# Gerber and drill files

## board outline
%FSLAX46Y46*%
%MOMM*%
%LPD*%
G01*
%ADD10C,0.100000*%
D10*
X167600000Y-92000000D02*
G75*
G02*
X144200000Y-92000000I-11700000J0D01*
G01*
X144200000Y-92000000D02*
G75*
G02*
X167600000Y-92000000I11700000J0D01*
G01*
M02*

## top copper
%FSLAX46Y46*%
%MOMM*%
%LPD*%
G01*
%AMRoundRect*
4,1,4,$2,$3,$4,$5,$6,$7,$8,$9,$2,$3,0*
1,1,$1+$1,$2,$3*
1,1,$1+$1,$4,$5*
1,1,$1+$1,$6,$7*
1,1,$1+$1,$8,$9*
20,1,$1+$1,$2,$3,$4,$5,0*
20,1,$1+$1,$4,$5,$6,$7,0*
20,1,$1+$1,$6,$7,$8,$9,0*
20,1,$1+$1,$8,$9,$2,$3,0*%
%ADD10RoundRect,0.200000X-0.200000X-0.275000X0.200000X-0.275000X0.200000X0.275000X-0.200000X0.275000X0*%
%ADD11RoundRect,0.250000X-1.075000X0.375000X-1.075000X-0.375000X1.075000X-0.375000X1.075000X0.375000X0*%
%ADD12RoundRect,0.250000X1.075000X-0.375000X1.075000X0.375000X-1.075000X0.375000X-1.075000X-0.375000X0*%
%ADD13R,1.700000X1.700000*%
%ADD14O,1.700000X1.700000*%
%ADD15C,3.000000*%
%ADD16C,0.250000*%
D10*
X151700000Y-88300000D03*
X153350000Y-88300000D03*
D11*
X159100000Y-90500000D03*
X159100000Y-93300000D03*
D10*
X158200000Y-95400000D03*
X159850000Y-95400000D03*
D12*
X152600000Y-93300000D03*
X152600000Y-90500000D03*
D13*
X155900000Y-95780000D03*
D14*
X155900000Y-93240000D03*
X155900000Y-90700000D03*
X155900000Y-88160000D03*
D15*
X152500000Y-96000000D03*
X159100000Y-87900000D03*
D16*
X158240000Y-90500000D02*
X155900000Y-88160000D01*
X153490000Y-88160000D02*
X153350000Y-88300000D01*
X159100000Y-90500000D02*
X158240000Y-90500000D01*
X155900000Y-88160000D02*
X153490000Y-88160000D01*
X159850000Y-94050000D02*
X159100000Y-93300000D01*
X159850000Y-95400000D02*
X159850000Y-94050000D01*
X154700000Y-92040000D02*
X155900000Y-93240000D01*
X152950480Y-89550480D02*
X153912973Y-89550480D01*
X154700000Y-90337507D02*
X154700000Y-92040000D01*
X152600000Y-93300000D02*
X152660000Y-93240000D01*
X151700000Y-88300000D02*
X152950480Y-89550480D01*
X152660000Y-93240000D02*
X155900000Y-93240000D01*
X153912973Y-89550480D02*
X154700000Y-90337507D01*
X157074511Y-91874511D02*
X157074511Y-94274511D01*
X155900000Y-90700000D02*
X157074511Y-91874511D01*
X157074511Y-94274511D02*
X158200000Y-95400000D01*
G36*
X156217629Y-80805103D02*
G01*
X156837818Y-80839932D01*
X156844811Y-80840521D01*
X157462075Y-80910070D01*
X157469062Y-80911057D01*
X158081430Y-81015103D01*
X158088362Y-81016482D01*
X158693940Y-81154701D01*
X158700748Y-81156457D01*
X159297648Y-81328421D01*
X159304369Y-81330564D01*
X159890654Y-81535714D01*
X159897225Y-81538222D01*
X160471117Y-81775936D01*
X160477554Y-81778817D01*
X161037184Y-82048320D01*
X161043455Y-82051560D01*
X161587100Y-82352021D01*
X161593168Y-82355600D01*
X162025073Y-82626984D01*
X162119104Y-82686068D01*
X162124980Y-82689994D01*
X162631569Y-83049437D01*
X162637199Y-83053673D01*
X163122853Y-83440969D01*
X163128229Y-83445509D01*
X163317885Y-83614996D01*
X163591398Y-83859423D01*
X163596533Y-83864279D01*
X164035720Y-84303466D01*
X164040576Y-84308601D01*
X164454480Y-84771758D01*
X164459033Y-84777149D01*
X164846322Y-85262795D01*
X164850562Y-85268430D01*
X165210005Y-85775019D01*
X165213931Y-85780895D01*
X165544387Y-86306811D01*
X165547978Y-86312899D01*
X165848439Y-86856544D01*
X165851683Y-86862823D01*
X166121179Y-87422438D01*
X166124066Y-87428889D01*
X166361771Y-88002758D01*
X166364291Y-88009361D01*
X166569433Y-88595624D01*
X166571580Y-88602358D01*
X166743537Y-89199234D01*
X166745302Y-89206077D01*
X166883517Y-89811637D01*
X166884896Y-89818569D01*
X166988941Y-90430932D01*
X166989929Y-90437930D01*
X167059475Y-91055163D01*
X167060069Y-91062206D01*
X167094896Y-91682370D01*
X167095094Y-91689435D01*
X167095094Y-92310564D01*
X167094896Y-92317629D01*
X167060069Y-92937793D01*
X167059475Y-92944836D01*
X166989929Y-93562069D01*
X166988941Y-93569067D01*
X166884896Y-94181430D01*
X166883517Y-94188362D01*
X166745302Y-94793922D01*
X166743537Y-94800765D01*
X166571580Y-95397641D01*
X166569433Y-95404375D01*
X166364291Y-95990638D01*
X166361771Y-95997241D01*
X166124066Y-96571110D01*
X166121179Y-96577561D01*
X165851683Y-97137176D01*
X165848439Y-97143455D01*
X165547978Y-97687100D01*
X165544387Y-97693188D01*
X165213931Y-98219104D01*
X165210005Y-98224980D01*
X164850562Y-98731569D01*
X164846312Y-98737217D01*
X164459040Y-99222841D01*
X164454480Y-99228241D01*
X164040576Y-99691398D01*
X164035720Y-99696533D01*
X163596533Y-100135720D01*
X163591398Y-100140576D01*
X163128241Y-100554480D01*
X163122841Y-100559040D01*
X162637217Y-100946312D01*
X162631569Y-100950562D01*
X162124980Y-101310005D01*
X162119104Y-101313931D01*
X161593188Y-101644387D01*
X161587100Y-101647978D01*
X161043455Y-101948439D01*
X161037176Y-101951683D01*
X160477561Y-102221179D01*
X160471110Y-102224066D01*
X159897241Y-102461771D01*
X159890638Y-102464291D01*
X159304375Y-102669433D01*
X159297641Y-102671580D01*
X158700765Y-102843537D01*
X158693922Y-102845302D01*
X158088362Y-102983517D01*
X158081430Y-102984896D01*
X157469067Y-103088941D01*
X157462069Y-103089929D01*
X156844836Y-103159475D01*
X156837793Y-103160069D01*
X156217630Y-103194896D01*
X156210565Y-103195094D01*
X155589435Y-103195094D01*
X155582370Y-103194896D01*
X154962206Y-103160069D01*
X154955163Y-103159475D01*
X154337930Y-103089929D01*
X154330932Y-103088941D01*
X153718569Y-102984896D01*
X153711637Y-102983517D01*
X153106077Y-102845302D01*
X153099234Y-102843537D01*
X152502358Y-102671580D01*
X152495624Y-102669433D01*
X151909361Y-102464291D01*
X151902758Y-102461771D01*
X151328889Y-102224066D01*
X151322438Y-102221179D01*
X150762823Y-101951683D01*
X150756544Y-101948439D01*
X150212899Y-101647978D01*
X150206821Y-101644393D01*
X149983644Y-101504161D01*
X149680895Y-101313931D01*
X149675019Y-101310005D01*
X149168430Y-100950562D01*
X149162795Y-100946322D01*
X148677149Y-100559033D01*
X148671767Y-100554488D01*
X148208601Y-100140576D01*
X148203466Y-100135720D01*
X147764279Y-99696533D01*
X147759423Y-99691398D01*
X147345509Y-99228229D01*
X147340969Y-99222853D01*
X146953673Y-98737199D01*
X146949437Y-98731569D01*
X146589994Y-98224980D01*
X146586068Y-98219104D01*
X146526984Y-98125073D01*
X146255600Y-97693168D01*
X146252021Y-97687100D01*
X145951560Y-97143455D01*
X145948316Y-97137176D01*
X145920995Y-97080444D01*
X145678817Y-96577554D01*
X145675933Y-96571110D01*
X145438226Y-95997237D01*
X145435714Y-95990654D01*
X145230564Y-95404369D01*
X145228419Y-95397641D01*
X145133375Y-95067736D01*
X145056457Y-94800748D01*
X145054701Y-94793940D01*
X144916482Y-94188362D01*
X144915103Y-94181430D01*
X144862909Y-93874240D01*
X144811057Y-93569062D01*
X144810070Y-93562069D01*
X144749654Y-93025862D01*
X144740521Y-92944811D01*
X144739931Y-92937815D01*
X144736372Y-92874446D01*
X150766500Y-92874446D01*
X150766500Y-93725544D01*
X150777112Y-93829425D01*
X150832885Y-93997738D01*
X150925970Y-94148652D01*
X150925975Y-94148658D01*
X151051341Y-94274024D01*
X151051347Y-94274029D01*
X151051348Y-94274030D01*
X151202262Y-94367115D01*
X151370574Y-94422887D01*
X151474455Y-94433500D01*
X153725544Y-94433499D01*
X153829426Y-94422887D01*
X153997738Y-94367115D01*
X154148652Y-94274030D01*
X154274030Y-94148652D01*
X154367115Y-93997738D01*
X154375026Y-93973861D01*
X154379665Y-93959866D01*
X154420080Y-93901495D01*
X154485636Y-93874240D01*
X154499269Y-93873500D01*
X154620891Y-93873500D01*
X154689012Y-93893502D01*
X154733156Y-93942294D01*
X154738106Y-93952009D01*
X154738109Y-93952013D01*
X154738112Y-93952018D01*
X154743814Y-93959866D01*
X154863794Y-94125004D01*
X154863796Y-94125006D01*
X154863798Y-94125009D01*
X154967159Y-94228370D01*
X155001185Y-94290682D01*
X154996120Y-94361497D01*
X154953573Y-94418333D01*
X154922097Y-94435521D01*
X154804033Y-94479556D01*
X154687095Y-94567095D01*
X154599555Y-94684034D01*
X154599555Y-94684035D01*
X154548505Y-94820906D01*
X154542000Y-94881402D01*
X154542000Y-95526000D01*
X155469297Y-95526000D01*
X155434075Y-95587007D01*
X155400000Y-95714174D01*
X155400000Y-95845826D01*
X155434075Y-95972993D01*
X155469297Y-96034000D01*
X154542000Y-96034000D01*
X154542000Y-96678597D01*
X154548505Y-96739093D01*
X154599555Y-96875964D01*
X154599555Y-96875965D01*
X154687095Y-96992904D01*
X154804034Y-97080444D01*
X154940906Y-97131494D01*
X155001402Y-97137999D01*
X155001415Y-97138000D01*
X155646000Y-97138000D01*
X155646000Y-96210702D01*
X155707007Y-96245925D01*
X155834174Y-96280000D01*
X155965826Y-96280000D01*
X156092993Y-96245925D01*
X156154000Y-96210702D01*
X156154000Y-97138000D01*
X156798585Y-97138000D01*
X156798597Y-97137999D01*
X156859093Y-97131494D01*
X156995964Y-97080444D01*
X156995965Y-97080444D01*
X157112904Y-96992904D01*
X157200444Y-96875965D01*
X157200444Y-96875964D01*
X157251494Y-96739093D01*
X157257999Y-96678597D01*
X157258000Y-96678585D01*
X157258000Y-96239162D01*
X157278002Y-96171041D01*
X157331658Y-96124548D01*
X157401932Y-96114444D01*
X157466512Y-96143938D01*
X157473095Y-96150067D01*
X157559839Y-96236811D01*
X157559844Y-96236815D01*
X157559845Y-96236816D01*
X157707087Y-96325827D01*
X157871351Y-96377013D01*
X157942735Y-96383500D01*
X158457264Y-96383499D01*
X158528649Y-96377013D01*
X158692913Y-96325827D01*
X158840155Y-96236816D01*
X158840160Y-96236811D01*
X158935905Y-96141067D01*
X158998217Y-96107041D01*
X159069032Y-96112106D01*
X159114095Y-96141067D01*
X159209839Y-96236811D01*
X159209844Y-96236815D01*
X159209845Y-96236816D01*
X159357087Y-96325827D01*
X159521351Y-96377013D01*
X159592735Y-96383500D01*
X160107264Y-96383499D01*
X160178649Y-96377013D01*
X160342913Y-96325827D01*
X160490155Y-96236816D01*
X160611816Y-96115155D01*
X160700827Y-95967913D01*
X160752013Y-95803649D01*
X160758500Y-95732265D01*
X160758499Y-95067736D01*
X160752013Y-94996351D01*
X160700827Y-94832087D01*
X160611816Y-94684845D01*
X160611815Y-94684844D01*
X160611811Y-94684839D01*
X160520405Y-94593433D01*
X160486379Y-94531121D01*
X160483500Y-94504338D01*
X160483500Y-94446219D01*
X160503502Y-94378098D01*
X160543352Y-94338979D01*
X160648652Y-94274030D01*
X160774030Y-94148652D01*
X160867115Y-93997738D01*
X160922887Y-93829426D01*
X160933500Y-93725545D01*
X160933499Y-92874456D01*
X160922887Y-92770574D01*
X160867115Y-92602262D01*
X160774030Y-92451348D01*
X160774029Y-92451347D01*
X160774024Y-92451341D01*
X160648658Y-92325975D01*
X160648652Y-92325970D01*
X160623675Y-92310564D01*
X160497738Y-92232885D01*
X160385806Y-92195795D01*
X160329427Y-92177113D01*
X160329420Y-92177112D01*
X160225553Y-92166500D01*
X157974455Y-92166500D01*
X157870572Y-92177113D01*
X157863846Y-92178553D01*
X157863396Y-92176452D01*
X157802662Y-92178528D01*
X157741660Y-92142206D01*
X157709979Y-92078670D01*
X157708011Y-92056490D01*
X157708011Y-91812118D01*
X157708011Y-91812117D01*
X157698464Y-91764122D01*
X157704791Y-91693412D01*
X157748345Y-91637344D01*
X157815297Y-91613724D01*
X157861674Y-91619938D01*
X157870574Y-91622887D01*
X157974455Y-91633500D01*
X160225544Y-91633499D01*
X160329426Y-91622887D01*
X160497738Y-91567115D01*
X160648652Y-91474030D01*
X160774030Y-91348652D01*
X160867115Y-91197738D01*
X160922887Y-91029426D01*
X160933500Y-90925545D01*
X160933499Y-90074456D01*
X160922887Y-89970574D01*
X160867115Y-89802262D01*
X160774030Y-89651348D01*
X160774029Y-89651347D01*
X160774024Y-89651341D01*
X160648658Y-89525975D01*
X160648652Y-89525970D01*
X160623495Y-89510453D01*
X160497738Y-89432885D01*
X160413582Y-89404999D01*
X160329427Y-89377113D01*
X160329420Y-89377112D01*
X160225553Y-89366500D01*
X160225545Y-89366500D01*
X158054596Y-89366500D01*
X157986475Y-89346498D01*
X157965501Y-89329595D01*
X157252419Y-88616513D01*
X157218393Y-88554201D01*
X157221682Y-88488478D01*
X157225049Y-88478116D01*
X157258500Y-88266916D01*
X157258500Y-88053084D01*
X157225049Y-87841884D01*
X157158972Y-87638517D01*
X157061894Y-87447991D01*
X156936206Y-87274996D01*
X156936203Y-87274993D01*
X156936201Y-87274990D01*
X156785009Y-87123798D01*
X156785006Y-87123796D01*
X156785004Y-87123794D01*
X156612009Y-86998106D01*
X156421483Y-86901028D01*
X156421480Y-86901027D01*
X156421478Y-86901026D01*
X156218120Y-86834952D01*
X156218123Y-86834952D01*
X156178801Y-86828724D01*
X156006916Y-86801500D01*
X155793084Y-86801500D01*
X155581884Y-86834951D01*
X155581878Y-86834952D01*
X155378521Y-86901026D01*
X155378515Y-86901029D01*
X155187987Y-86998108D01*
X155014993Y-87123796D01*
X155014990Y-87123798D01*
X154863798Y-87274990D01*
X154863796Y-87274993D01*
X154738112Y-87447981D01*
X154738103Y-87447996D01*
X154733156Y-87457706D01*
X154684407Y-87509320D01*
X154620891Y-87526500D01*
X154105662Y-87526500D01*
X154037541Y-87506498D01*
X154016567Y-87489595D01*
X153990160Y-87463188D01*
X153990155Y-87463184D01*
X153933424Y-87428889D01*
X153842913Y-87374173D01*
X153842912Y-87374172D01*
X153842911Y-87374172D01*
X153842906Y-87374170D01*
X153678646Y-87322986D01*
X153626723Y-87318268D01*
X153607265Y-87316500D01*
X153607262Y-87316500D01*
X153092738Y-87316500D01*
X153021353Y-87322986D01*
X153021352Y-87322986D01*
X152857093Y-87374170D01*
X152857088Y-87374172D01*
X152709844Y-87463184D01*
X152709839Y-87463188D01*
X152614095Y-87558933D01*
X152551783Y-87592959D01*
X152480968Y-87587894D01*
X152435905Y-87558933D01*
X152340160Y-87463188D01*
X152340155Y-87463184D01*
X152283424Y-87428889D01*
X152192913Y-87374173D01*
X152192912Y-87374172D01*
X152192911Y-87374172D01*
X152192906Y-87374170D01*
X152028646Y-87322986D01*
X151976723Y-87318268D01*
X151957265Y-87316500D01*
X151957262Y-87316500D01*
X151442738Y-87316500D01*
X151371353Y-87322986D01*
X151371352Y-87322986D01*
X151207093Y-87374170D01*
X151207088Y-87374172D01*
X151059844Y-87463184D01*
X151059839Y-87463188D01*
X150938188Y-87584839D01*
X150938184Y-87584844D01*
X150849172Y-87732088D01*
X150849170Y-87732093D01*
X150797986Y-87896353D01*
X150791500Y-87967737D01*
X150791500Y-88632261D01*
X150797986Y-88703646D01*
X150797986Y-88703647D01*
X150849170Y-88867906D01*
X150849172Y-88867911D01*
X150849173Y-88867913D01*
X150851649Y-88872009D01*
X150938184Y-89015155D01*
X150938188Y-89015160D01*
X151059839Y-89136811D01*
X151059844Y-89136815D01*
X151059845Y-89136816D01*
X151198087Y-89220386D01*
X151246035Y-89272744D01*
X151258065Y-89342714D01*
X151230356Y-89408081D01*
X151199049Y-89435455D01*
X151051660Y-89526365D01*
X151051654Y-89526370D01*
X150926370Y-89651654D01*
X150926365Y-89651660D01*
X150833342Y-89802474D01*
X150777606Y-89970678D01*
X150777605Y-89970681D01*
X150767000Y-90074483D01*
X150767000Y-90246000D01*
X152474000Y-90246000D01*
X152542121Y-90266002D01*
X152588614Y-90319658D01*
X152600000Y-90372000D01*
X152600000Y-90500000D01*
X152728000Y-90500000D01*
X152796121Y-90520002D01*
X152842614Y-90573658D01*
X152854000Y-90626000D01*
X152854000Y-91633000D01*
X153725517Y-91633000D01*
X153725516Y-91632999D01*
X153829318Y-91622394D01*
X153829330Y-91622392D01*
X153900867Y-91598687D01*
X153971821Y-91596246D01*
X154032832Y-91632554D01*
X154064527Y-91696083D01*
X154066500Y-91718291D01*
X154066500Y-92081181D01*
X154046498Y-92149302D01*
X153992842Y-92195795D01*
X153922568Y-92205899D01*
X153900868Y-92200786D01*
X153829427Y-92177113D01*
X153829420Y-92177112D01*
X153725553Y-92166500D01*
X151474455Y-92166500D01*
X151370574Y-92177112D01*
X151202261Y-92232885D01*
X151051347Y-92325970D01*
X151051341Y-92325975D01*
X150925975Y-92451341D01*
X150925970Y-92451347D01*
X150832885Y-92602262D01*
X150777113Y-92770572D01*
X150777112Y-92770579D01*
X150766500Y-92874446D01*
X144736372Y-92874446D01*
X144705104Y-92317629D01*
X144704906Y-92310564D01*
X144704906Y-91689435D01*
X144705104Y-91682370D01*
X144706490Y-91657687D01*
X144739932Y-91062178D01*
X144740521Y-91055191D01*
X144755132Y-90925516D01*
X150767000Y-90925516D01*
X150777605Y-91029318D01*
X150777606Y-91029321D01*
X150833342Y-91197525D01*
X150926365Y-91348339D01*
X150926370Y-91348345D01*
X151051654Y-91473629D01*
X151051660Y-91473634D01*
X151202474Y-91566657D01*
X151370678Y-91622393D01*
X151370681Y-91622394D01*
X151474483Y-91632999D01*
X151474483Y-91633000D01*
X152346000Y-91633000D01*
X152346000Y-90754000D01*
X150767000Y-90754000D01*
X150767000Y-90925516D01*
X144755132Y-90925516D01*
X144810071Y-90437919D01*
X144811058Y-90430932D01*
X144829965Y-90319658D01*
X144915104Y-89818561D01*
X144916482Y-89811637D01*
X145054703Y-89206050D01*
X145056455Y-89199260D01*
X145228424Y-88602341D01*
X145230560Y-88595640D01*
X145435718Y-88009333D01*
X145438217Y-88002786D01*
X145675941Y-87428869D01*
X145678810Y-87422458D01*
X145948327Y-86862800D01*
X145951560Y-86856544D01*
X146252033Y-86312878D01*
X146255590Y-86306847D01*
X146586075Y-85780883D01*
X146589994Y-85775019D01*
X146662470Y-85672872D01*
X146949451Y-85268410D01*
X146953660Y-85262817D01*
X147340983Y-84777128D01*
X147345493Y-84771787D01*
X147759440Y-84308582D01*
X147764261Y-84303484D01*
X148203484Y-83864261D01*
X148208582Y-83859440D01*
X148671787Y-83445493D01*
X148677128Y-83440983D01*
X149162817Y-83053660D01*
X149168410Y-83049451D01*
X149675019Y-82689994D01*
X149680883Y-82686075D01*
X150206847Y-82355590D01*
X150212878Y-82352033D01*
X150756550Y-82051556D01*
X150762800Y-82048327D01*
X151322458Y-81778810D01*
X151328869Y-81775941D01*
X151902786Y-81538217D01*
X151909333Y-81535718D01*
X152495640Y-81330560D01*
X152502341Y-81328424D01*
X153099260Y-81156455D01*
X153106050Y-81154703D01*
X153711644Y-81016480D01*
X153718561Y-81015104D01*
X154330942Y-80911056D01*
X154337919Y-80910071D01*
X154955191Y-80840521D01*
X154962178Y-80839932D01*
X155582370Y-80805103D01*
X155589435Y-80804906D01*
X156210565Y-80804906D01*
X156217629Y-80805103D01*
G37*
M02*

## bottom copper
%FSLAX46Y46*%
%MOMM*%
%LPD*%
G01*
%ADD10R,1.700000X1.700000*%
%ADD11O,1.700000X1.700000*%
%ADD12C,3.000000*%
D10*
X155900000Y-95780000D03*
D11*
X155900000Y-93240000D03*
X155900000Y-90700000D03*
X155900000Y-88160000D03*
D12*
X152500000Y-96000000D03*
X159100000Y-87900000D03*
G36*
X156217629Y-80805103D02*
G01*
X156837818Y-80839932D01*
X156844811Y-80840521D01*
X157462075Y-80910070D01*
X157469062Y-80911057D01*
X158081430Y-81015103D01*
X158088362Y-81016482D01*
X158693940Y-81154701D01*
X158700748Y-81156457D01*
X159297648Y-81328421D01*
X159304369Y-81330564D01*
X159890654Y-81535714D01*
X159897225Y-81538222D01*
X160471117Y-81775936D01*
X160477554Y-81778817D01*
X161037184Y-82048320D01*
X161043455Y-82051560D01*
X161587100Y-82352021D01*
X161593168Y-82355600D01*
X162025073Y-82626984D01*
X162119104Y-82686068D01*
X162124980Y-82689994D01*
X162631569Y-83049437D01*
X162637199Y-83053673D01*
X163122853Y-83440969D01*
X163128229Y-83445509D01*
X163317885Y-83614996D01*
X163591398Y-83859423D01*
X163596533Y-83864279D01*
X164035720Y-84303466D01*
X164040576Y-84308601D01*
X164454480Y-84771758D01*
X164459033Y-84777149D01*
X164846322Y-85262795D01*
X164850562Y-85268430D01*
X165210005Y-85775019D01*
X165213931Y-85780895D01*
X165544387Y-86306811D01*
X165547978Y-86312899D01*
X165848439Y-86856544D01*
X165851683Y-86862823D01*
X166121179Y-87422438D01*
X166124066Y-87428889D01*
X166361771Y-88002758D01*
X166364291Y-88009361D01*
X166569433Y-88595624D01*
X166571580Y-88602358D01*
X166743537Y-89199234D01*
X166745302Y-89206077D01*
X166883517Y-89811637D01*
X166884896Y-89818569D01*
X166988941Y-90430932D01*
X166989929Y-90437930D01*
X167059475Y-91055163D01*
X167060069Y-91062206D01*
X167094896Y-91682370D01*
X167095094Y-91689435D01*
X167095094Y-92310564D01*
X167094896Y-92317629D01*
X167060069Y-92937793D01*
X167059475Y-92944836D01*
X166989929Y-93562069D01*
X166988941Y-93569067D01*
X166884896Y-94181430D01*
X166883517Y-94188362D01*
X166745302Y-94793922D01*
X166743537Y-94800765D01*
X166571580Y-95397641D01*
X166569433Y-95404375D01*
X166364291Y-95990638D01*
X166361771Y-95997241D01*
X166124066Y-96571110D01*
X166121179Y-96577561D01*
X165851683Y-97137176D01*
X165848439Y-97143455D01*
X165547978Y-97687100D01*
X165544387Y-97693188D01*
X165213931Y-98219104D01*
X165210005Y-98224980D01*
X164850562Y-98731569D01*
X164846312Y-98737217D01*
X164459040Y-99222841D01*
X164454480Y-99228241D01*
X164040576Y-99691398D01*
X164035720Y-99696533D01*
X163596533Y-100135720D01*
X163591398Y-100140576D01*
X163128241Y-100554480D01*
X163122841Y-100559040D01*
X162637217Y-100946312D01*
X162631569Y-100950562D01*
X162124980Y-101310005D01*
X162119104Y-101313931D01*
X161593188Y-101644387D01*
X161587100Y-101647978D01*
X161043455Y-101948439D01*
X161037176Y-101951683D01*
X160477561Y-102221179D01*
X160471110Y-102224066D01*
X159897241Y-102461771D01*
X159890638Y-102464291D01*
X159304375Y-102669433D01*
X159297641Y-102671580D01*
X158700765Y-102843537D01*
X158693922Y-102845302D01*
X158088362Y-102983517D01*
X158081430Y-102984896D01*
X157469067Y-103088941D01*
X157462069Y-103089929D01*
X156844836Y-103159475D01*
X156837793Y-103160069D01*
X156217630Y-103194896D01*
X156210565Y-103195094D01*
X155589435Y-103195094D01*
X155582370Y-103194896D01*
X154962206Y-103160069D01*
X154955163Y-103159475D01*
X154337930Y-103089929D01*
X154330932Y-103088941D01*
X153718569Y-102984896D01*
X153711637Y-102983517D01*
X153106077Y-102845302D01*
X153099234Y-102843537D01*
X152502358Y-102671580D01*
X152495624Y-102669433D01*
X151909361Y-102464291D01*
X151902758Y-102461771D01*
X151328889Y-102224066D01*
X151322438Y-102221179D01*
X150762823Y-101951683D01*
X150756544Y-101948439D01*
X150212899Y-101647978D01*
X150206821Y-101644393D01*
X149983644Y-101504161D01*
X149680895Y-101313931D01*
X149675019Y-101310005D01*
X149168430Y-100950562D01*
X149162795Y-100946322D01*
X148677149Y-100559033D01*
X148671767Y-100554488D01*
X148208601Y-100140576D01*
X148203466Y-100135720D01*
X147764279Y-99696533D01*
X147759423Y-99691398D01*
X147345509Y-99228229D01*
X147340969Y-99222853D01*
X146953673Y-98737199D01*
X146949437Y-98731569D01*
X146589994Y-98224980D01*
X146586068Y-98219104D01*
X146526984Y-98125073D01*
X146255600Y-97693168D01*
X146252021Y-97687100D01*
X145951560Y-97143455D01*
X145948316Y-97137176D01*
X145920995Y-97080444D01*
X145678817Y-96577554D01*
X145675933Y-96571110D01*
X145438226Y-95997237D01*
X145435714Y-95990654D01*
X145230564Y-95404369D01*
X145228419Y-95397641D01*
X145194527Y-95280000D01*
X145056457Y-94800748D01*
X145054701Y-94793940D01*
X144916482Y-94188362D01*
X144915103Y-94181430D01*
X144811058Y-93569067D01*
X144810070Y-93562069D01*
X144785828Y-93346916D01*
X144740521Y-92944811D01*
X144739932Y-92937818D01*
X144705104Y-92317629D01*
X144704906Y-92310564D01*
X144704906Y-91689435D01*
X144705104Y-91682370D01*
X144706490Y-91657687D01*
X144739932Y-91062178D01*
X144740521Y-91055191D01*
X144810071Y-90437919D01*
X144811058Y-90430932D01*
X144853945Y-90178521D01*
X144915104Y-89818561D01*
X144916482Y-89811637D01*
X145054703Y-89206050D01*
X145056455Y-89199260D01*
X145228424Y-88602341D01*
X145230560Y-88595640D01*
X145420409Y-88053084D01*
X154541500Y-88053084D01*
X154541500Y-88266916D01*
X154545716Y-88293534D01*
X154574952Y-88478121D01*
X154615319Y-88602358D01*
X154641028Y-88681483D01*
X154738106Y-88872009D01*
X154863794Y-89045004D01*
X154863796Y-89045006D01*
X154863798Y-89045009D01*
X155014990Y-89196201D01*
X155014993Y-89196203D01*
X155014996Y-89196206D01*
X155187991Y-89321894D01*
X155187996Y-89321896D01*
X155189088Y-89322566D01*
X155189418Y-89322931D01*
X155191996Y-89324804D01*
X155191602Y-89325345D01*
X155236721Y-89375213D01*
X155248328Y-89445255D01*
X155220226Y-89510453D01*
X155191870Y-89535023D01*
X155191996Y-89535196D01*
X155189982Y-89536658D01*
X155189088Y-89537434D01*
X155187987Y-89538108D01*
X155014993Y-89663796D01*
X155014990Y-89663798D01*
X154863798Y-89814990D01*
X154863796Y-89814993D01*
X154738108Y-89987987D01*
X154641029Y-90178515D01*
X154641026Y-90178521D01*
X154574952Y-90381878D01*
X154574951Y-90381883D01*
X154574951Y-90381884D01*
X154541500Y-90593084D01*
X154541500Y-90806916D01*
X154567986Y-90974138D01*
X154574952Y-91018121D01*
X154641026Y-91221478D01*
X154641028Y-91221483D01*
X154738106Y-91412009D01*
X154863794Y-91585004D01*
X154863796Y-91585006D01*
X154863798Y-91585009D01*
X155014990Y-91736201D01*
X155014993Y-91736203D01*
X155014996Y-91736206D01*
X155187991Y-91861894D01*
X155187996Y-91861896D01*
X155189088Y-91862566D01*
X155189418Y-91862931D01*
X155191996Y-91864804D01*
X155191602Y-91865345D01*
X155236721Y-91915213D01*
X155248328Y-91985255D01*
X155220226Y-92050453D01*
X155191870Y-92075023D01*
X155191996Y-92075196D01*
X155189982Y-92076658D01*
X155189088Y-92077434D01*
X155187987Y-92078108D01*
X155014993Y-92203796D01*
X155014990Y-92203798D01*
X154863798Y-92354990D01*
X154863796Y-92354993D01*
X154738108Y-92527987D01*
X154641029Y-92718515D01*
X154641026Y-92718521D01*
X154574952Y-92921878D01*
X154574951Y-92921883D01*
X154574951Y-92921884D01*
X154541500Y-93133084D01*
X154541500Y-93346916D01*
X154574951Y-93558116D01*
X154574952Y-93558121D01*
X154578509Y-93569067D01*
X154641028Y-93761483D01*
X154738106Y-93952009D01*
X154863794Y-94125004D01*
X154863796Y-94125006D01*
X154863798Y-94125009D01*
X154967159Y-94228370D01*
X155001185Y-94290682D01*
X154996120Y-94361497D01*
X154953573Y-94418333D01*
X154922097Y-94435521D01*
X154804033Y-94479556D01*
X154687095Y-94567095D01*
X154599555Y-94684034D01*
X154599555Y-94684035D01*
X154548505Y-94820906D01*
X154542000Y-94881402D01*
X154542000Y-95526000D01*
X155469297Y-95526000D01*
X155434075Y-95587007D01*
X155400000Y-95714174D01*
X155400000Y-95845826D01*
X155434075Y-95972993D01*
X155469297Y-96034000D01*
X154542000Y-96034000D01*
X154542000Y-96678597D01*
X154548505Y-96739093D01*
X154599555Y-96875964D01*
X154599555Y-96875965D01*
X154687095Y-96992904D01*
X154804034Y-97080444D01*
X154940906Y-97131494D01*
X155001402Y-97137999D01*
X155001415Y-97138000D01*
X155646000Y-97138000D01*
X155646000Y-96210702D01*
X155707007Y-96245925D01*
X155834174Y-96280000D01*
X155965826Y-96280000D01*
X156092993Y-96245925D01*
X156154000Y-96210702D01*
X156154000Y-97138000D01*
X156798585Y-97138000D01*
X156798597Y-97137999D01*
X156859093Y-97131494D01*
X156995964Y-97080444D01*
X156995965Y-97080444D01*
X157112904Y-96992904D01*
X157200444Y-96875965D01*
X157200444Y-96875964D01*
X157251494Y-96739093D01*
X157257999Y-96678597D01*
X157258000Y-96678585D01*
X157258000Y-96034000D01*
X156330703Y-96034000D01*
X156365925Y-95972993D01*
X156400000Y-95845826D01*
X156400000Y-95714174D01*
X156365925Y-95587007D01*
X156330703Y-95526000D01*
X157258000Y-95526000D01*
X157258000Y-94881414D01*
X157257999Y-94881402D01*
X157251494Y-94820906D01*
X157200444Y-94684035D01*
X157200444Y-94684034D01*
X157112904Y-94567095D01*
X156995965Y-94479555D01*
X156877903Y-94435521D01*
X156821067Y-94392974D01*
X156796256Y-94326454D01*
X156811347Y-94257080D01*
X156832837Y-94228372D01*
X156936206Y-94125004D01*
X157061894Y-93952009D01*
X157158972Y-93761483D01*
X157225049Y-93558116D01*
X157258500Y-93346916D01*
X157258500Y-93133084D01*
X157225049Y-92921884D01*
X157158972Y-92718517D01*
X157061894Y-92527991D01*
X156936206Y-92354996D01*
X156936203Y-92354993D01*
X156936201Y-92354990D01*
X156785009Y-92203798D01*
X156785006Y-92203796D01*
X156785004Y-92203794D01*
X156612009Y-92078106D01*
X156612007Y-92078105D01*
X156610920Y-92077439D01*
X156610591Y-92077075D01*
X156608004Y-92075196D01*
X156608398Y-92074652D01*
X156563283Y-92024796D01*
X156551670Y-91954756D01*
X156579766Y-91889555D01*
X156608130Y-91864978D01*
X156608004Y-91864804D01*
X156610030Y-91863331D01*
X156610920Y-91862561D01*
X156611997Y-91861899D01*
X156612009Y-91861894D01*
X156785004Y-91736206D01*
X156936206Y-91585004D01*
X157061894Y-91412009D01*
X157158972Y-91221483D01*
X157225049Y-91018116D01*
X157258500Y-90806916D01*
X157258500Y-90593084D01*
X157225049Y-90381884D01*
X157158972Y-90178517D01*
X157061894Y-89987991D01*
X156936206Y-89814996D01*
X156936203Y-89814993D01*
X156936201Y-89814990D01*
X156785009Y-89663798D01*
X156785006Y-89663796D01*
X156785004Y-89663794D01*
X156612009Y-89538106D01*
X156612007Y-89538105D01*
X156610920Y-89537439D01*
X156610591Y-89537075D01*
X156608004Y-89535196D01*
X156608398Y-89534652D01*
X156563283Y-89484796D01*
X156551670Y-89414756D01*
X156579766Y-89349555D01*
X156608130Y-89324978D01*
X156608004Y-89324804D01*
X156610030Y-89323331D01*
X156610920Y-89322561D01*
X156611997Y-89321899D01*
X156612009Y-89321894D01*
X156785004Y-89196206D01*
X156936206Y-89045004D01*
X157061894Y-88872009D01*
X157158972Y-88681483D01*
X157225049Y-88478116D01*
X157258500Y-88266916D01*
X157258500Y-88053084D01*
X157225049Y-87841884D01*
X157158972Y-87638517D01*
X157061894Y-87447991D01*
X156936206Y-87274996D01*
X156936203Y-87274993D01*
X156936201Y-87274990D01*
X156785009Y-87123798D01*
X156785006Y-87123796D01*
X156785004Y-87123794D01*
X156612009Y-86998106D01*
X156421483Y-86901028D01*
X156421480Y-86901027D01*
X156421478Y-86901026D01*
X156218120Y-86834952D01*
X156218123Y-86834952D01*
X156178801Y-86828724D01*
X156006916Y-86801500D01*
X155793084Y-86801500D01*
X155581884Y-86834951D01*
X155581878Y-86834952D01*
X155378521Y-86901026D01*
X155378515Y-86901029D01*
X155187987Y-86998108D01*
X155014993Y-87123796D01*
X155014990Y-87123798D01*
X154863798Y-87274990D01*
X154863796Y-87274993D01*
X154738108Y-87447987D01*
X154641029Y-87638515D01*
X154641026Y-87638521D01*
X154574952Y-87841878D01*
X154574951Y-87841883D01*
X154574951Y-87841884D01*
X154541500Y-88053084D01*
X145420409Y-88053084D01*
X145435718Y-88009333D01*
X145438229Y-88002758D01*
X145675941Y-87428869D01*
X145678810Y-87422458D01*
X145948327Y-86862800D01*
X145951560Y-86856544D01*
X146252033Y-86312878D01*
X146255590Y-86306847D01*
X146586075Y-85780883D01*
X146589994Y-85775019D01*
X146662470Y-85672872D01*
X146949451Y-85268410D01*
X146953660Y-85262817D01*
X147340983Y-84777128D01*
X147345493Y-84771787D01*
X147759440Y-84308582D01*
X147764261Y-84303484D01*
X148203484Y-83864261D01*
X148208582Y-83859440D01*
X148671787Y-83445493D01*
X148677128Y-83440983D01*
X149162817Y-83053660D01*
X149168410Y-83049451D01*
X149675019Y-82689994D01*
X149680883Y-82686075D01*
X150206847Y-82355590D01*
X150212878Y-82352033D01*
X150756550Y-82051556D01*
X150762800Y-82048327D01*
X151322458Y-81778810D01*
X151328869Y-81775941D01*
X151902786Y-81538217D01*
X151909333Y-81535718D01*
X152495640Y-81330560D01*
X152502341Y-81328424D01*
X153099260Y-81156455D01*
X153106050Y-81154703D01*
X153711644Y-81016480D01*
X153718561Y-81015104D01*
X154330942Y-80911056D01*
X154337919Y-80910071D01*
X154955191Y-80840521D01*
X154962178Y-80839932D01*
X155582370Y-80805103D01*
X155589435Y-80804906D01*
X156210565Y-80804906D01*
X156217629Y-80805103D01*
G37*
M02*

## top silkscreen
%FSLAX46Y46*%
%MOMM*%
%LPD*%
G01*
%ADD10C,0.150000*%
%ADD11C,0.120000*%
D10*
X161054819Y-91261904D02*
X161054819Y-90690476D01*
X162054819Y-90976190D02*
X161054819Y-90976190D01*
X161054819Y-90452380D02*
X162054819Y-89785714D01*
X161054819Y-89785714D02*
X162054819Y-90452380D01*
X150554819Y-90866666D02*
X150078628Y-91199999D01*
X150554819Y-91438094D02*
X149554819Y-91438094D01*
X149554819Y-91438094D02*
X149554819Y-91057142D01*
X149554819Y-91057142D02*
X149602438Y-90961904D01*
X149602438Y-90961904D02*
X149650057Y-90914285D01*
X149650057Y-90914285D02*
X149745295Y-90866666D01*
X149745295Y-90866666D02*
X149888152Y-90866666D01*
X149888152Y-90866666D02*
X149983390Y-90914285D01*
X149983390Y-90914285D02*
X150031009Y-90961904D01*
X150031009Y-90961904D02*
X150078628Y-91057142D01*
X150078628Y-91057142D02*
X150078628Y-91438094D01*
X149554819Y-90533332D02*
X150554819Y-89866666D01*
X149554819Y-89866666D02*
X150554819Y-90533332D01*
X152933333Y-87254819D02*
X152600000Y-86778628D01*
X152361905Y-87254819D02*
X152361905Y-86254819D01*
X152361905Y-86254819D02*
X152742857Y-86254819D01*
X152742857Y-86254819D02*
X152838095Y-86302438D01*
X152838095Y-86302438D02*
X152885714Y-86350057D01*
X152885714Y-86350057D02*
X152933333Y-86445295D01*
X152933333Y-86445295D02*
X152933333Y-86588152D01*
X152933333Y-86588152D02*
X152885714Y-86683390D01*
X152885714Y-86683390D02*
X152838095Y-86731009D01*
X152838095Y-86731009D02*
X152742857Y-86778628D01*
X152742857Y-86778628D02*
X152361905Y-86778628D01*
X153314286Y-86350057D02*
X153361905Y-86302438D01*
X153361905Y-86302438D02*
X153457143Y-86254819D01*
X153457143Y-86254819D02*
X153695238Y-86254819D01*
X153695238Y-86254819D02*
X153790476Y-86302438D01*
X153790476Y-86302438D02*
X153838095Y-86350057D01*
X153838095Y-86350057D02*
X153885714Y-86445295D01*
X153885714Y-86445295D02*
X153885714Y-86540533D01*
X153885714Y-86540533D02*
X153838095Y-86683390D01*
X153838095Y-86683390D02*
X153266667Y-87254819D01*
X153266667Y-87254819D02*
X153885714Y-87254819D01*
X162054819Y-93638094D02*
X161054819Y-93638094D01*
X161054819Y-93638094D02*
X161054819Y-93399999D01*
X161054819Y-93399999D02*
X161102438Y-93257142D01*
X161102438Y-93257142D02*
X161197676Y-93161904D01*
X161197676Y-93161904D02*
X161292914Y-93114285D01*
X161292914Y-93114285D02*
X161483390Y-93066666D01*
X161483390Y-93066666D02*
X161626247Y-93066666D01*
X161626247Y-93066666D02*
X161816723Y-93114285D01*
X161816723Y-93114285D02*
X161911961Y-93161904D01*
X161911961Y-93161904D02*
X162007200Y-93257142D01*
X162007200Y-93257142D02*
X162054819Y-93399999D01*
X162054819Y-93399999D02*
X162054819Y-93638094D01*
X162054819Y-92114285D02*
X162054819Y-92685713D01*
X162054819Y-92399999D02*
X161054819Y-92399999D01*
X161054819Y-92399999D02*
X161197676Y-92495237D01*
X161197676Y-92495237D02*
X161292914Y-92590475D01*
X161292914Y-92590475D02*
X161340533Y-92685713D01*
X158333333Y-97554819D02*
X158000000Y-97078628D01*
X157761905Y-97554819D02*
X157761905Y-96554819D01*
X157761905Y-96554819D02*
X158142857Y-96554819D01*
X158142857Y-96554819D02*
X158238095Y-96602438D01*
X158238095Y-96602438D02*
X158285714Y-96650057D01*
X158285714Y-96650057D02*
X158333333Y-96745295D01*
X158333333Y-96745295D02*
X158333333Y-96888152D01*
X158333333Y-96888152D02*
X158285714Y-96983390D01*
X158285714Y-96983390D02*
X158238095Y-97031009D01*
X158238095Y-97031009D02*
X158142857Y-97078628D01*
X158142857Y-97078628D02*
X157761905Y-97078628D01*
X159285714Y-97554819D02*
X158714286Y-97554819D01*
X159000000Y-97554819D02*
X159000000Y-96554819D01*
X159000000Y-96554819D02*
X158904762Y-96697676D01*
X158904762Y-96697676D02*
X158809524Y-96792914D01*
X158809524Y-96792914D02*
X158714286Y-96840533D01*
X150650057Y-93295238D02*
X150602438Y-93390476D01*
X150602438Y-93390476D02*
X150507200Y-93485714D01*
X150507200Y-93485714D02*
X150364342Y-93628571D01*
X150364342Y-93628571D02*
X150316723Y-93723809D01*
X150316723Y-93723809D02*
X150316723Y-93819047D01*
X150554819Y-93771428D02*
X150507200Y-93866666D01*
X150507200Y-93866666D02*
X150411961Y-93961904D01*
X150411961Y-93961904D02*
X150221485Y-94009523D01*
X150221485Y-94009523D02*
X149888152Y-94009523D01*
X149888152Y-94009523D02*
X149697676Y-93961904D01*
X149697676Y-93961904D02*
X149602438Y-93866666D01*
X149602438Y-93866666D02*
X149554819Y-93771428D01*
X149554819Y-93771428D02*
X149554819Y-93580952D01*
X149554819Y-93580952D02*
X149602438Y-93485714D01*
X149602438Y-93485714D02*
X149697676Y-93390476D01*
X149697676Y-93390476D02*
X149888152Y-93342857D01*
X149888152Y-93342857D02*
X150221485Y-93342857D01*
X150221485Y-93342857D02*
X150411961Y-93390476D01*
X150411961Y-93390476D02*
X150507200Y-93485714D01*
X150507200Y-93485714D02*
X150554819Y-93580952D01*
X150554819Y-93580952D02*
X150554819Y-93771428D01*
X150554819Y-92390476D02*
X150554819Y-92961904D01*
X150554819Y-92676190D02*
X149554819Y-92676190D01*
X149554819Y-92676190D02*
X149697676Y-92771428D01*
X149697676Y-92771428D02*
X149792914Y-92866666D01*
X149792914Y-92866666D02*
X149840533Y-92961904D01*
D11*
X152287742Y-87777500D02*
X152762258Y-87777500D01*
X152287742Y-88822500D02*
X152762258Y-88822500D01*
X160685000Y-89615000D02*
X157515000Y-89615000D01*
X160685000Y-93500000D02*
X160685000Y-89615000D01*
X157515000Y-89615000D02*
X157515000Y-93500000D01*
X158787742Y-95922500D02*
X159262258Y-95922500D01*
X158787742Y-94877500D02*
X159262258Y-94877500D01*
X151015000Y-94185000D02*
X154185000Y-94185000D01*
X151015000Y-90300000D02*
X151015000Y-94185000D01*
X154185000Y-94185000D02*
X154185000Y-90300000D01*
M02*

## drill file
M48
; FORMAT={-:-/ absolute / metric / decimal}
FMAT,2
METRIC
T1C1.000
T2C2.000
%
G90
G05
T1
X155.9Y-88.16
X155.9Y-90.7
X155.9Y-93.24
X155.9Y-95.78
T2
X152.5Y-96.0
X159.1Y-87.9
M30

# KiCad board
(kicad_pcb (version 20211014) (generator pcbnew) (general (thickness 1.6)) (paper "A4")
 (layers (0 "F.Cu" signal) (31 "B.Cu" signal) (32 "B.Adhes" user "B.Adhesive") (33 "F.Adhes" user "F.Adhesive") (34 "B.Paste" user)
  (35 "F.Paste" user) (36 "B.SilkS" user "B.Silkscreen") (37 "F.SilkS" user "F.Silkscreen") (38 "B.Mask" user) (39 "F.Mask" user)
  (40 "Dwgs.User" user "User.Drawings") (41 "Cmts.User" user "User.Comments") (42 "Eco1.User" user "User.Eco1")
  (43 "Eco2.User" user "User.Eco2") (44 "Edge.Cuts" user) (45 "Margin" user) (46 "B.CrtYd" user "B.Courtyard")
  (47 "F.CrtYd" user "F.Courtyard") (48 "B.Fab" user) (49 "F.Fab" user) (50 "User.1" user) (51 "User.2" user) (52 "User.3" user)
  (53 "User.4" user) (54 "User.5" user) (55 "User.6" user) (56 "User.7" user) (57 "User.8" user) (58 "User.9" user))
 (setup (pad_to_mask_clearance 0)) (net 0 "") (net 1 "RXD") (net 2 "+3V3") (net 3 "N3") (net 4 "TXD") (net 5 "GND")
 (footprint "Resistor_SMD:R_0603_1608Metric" (layer "F.Cu") (at 152.525 88.3)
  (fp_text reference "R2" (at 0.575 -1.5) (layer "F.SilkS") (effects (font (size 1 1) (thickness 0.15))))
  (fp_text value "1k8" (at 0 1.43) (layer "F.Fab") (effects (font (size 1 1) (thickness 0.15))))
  (fp_line (start -0.237258 -0.5225) (end 0.237258 -0.5225) (layer "F.SilkS") (width 0.12))
  (fp_line (start -0.237258 0.5225) (end 0.237258 0.5225) (layer "F.SilkS") (width 0.12))
  (pad "1" smd roundrect locked (at -0.825 0) (size 0.8 0.95) (layers "F.Cu" "F.Paste" "F.Mask") (roundrect_rratio 0.25) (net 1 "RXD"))
  (pad "2" smd roundrect locked (at 0.825 0) (size 0.8 0.95) (layers "F.Cu" "F.Paste" "F.Mask") (roundrect_rratio 0.25) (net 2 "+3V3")))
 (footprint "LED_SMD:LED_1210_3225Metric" (layer "F.Cu") (at 159.1 91.9 -90)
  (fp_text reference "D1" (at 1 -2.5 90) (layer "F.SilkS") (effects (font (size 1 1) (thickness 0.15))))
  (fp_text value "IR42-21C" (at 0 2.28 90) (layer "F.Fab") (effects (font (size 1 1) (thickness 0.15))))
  (fp_line (start -2.285 -1.585) (end -2.285 1.585) (layer "F.SilkS") (width 0.12))
  (fp_line (start 1.6 -1.585) (end -2.285 -1.585) (layer "F.SilkS") (width 0.12))
  (fp_line (start -2.285 1.585) (end 1.6 1.585) (layer "F.SilkS") (width 0.12))
  (pad "1" smd roundrect locked (at -1.4 0 270) (size 1.25 2.65) (layers "F.Cu" "F.Paste" "F.Mask") (roundrect_rratio 0.2) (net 2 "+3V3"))
  (pad "2" smd roundrect locked (at 1.4 0 270) (size 1.25 2.65) (layers "F.Cu" "F.Paste" "F.Mask") (roundrect_rratio 0.2) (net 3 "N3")))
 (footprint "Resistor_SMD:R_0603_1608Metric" (layer "F.Cu") (at 159.025 95.4)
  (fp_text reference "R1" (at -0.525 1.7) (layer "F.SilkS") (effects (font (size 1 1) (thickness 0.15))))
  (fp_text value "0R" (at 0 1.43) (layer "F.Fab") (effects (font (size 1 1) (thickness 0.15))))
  (fp_line (start -0.237258 0.5225) (end 0.237258 0.5225) (layer "F.SilkS") (width 0.12))
  (fp_line (start -0.237258 -0.5225) (end 0.237258 -0.5225) (layer "F.SilkS") (width 0.12))
  (pad "1" smd roundrect locked (at -0.825 0) (size 0.8 0.95) (layers "F.Cu" "F.Paste" "F.Mask") (roundrect_rratio 0.25) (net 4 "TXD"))
  (pad "2" smd roundrect locked (at 0.825 0) (size 0.8 0.95) (layers "F.Cu" "F.Paste" "F.Mask") (roundrect_rratio 0.25) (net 3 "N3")))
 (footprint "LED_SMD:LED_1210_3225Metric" (layer "F.Cu") (at 152.6 91.9 90)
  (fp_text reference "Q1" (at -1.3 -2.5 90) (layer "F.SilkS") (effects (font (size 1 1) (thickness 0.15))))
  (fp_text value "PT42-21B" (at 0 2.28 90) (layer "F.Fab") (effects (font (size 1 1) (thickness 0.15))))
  (fp_line (start -2.285 -1.585) (end -2.285 1.585) (layer "F.SilkS") (width 0.12))
  (fp_line (start 1.6 -1.585) (end -2.285 -1.585) (layer "F.SilkS") (width 0.12))
  (fp_line (start -2.285 1.585) (end 1.6 1.585) (layer "F.SilkS") (width 0.12))
  (pad "1" smd roundrect locked (at -1.4 0 90) (size 1.25 2.65) (layers "F.Cu" "F.Paste" "F.Mask") (roundrect_rratio 0.2) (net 1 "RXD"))
  (pad "2" smd roundrect locked (at 1.4 0 90) (size 1.25 2.65) (layers "F.Cu" "F.Paste" "F.Mask") (roundrect_rratio 0.2) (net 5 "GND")))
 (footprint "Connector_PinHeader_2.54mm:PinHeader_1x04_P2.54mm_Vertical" (layer "B.Cu") (at 155.9 95.78)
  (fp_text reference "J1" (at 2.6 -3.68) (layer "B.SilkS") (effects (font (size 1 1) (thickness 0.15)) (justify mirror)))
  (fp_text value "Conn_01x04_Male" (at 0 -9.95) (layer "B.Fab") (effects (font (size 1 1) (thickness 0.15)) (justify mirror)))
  (pad "1" thru_hole rect locked (at 0 0) (size 1.7 1.7) (drill 1) (layers *.Cu *.Mask) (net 5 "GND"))
  (pad "2" thru_hole oval locked (at 0 -2.54) (size 1.7 1.7) (drill 1) (layers *.Cu *.Mask) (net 1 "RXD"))
  (pad "3" thru_hole oval locked (at 0 -5.08) (size 1.7 1.7) (drill 1) (layers *.Cu *.Mask) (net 4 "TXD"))
  (pad "4" thru_hole oval locked (at 0 -7.62) (size 1.7 1.7) (drill 1) (layers *.Cu *.Mask) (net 2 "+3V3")))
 (gr_circle (center 155.9 92) (end 167.6 92) (layer "Edge.Cuts") (width 0.1) (fill none))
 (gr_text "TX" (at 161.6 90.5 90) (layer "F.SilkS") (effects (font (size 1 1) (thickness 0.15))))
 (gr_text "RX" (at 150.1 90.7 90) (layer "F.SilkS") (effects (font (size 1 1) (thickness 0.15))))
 (segment (start 158.24 90.5) (end 155.9 88.16) (width 0.25) (layer "F.Cu") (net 2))
 (segment (start 153.49 88.16) (end 153.35 88.3) (width 0.25) (layer "F.Cu") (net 2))
 (segment (start 159.1 90.5) (end 158.24 90.5) (width 0.25) (layer "F.Cu") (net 2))
 (segment (start 155.9 88.16) (end 153.49 88.16) (width 0.25) (layer "F.Cu") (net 2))
 (segment (start 159.85 94.05) (end 159.1 93.3) (width 0.25) (layer "F.Cu") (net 3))
 (segment (start 159.85 95.4) (end 159.85 94.05) (width 0.25) (layer "F.Cu") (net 3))
 (segment (start 154.7 92.04) (end 155.9 93.24) (width 0.25) (layer "F.Cu") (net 1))
 (segment (start 152.95048 89.55048) (end 153.912973 89.55048) (width 0.25) (layer "F.Cu") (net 1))
 (segment (start 154.7 90.337507) (end 154.7 92.04) (width 0.25) (layer "F.Cu") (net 1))
 (segment (start 152.6 93.3) (end 152.66 93.24) (width 0.25) (layer "F.Cu") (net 1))
 (segment (start 151.7 88.3) (end 152.95048 89.55048) (width 0.25) (layer "F.Cu") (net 1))
 (segment (start 152.66 93.24) (end 155.9 93.24) (width 0.25) (layer "F.Cu") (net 1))
 (segment (start 153.912973 89.55048) (end 154.7 90.337507) (width 0.25) (layer "F.Cu") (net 1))
 (segment (start 157.074511 91.874511) (end 157.074511 94.274511) (width 0.25) (layer "F.Cu") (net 4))
 (segment (start 155.9 90.7) (end 157.074511 91.874511) (width 0.25) (layer "F.Cu") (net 4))
 (segment (start 157.074511 94.274511) (end 158.2 95.4) (width 0.25) (layer "F.Cu") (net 4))
 (via (at 152.5 96) (size 3) (drill 2) (layers "F.Cu" "B.Cu") (free) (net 5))
 (via (at 159.1 87.9) (size 3) (drill 2) (layers "F.Cu" "B.Cu") (free) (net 5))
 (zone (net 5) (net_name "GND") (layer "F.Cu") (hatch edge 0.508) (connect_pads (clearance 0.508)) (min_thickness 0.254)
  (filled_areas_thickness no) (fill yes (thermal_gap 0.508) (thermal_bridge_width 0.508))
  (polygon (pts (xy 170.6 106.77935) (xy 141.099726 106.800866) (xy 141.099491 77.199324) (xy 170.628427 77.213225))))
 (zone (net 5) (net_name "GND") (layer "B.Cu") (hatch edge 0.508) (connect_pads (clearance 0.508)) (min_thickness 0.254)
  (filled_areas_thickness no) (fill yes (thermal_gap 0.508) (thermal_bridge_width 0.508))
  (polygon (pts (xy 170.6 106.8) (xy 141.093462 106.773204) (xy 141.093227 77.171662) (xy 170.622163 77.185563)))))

